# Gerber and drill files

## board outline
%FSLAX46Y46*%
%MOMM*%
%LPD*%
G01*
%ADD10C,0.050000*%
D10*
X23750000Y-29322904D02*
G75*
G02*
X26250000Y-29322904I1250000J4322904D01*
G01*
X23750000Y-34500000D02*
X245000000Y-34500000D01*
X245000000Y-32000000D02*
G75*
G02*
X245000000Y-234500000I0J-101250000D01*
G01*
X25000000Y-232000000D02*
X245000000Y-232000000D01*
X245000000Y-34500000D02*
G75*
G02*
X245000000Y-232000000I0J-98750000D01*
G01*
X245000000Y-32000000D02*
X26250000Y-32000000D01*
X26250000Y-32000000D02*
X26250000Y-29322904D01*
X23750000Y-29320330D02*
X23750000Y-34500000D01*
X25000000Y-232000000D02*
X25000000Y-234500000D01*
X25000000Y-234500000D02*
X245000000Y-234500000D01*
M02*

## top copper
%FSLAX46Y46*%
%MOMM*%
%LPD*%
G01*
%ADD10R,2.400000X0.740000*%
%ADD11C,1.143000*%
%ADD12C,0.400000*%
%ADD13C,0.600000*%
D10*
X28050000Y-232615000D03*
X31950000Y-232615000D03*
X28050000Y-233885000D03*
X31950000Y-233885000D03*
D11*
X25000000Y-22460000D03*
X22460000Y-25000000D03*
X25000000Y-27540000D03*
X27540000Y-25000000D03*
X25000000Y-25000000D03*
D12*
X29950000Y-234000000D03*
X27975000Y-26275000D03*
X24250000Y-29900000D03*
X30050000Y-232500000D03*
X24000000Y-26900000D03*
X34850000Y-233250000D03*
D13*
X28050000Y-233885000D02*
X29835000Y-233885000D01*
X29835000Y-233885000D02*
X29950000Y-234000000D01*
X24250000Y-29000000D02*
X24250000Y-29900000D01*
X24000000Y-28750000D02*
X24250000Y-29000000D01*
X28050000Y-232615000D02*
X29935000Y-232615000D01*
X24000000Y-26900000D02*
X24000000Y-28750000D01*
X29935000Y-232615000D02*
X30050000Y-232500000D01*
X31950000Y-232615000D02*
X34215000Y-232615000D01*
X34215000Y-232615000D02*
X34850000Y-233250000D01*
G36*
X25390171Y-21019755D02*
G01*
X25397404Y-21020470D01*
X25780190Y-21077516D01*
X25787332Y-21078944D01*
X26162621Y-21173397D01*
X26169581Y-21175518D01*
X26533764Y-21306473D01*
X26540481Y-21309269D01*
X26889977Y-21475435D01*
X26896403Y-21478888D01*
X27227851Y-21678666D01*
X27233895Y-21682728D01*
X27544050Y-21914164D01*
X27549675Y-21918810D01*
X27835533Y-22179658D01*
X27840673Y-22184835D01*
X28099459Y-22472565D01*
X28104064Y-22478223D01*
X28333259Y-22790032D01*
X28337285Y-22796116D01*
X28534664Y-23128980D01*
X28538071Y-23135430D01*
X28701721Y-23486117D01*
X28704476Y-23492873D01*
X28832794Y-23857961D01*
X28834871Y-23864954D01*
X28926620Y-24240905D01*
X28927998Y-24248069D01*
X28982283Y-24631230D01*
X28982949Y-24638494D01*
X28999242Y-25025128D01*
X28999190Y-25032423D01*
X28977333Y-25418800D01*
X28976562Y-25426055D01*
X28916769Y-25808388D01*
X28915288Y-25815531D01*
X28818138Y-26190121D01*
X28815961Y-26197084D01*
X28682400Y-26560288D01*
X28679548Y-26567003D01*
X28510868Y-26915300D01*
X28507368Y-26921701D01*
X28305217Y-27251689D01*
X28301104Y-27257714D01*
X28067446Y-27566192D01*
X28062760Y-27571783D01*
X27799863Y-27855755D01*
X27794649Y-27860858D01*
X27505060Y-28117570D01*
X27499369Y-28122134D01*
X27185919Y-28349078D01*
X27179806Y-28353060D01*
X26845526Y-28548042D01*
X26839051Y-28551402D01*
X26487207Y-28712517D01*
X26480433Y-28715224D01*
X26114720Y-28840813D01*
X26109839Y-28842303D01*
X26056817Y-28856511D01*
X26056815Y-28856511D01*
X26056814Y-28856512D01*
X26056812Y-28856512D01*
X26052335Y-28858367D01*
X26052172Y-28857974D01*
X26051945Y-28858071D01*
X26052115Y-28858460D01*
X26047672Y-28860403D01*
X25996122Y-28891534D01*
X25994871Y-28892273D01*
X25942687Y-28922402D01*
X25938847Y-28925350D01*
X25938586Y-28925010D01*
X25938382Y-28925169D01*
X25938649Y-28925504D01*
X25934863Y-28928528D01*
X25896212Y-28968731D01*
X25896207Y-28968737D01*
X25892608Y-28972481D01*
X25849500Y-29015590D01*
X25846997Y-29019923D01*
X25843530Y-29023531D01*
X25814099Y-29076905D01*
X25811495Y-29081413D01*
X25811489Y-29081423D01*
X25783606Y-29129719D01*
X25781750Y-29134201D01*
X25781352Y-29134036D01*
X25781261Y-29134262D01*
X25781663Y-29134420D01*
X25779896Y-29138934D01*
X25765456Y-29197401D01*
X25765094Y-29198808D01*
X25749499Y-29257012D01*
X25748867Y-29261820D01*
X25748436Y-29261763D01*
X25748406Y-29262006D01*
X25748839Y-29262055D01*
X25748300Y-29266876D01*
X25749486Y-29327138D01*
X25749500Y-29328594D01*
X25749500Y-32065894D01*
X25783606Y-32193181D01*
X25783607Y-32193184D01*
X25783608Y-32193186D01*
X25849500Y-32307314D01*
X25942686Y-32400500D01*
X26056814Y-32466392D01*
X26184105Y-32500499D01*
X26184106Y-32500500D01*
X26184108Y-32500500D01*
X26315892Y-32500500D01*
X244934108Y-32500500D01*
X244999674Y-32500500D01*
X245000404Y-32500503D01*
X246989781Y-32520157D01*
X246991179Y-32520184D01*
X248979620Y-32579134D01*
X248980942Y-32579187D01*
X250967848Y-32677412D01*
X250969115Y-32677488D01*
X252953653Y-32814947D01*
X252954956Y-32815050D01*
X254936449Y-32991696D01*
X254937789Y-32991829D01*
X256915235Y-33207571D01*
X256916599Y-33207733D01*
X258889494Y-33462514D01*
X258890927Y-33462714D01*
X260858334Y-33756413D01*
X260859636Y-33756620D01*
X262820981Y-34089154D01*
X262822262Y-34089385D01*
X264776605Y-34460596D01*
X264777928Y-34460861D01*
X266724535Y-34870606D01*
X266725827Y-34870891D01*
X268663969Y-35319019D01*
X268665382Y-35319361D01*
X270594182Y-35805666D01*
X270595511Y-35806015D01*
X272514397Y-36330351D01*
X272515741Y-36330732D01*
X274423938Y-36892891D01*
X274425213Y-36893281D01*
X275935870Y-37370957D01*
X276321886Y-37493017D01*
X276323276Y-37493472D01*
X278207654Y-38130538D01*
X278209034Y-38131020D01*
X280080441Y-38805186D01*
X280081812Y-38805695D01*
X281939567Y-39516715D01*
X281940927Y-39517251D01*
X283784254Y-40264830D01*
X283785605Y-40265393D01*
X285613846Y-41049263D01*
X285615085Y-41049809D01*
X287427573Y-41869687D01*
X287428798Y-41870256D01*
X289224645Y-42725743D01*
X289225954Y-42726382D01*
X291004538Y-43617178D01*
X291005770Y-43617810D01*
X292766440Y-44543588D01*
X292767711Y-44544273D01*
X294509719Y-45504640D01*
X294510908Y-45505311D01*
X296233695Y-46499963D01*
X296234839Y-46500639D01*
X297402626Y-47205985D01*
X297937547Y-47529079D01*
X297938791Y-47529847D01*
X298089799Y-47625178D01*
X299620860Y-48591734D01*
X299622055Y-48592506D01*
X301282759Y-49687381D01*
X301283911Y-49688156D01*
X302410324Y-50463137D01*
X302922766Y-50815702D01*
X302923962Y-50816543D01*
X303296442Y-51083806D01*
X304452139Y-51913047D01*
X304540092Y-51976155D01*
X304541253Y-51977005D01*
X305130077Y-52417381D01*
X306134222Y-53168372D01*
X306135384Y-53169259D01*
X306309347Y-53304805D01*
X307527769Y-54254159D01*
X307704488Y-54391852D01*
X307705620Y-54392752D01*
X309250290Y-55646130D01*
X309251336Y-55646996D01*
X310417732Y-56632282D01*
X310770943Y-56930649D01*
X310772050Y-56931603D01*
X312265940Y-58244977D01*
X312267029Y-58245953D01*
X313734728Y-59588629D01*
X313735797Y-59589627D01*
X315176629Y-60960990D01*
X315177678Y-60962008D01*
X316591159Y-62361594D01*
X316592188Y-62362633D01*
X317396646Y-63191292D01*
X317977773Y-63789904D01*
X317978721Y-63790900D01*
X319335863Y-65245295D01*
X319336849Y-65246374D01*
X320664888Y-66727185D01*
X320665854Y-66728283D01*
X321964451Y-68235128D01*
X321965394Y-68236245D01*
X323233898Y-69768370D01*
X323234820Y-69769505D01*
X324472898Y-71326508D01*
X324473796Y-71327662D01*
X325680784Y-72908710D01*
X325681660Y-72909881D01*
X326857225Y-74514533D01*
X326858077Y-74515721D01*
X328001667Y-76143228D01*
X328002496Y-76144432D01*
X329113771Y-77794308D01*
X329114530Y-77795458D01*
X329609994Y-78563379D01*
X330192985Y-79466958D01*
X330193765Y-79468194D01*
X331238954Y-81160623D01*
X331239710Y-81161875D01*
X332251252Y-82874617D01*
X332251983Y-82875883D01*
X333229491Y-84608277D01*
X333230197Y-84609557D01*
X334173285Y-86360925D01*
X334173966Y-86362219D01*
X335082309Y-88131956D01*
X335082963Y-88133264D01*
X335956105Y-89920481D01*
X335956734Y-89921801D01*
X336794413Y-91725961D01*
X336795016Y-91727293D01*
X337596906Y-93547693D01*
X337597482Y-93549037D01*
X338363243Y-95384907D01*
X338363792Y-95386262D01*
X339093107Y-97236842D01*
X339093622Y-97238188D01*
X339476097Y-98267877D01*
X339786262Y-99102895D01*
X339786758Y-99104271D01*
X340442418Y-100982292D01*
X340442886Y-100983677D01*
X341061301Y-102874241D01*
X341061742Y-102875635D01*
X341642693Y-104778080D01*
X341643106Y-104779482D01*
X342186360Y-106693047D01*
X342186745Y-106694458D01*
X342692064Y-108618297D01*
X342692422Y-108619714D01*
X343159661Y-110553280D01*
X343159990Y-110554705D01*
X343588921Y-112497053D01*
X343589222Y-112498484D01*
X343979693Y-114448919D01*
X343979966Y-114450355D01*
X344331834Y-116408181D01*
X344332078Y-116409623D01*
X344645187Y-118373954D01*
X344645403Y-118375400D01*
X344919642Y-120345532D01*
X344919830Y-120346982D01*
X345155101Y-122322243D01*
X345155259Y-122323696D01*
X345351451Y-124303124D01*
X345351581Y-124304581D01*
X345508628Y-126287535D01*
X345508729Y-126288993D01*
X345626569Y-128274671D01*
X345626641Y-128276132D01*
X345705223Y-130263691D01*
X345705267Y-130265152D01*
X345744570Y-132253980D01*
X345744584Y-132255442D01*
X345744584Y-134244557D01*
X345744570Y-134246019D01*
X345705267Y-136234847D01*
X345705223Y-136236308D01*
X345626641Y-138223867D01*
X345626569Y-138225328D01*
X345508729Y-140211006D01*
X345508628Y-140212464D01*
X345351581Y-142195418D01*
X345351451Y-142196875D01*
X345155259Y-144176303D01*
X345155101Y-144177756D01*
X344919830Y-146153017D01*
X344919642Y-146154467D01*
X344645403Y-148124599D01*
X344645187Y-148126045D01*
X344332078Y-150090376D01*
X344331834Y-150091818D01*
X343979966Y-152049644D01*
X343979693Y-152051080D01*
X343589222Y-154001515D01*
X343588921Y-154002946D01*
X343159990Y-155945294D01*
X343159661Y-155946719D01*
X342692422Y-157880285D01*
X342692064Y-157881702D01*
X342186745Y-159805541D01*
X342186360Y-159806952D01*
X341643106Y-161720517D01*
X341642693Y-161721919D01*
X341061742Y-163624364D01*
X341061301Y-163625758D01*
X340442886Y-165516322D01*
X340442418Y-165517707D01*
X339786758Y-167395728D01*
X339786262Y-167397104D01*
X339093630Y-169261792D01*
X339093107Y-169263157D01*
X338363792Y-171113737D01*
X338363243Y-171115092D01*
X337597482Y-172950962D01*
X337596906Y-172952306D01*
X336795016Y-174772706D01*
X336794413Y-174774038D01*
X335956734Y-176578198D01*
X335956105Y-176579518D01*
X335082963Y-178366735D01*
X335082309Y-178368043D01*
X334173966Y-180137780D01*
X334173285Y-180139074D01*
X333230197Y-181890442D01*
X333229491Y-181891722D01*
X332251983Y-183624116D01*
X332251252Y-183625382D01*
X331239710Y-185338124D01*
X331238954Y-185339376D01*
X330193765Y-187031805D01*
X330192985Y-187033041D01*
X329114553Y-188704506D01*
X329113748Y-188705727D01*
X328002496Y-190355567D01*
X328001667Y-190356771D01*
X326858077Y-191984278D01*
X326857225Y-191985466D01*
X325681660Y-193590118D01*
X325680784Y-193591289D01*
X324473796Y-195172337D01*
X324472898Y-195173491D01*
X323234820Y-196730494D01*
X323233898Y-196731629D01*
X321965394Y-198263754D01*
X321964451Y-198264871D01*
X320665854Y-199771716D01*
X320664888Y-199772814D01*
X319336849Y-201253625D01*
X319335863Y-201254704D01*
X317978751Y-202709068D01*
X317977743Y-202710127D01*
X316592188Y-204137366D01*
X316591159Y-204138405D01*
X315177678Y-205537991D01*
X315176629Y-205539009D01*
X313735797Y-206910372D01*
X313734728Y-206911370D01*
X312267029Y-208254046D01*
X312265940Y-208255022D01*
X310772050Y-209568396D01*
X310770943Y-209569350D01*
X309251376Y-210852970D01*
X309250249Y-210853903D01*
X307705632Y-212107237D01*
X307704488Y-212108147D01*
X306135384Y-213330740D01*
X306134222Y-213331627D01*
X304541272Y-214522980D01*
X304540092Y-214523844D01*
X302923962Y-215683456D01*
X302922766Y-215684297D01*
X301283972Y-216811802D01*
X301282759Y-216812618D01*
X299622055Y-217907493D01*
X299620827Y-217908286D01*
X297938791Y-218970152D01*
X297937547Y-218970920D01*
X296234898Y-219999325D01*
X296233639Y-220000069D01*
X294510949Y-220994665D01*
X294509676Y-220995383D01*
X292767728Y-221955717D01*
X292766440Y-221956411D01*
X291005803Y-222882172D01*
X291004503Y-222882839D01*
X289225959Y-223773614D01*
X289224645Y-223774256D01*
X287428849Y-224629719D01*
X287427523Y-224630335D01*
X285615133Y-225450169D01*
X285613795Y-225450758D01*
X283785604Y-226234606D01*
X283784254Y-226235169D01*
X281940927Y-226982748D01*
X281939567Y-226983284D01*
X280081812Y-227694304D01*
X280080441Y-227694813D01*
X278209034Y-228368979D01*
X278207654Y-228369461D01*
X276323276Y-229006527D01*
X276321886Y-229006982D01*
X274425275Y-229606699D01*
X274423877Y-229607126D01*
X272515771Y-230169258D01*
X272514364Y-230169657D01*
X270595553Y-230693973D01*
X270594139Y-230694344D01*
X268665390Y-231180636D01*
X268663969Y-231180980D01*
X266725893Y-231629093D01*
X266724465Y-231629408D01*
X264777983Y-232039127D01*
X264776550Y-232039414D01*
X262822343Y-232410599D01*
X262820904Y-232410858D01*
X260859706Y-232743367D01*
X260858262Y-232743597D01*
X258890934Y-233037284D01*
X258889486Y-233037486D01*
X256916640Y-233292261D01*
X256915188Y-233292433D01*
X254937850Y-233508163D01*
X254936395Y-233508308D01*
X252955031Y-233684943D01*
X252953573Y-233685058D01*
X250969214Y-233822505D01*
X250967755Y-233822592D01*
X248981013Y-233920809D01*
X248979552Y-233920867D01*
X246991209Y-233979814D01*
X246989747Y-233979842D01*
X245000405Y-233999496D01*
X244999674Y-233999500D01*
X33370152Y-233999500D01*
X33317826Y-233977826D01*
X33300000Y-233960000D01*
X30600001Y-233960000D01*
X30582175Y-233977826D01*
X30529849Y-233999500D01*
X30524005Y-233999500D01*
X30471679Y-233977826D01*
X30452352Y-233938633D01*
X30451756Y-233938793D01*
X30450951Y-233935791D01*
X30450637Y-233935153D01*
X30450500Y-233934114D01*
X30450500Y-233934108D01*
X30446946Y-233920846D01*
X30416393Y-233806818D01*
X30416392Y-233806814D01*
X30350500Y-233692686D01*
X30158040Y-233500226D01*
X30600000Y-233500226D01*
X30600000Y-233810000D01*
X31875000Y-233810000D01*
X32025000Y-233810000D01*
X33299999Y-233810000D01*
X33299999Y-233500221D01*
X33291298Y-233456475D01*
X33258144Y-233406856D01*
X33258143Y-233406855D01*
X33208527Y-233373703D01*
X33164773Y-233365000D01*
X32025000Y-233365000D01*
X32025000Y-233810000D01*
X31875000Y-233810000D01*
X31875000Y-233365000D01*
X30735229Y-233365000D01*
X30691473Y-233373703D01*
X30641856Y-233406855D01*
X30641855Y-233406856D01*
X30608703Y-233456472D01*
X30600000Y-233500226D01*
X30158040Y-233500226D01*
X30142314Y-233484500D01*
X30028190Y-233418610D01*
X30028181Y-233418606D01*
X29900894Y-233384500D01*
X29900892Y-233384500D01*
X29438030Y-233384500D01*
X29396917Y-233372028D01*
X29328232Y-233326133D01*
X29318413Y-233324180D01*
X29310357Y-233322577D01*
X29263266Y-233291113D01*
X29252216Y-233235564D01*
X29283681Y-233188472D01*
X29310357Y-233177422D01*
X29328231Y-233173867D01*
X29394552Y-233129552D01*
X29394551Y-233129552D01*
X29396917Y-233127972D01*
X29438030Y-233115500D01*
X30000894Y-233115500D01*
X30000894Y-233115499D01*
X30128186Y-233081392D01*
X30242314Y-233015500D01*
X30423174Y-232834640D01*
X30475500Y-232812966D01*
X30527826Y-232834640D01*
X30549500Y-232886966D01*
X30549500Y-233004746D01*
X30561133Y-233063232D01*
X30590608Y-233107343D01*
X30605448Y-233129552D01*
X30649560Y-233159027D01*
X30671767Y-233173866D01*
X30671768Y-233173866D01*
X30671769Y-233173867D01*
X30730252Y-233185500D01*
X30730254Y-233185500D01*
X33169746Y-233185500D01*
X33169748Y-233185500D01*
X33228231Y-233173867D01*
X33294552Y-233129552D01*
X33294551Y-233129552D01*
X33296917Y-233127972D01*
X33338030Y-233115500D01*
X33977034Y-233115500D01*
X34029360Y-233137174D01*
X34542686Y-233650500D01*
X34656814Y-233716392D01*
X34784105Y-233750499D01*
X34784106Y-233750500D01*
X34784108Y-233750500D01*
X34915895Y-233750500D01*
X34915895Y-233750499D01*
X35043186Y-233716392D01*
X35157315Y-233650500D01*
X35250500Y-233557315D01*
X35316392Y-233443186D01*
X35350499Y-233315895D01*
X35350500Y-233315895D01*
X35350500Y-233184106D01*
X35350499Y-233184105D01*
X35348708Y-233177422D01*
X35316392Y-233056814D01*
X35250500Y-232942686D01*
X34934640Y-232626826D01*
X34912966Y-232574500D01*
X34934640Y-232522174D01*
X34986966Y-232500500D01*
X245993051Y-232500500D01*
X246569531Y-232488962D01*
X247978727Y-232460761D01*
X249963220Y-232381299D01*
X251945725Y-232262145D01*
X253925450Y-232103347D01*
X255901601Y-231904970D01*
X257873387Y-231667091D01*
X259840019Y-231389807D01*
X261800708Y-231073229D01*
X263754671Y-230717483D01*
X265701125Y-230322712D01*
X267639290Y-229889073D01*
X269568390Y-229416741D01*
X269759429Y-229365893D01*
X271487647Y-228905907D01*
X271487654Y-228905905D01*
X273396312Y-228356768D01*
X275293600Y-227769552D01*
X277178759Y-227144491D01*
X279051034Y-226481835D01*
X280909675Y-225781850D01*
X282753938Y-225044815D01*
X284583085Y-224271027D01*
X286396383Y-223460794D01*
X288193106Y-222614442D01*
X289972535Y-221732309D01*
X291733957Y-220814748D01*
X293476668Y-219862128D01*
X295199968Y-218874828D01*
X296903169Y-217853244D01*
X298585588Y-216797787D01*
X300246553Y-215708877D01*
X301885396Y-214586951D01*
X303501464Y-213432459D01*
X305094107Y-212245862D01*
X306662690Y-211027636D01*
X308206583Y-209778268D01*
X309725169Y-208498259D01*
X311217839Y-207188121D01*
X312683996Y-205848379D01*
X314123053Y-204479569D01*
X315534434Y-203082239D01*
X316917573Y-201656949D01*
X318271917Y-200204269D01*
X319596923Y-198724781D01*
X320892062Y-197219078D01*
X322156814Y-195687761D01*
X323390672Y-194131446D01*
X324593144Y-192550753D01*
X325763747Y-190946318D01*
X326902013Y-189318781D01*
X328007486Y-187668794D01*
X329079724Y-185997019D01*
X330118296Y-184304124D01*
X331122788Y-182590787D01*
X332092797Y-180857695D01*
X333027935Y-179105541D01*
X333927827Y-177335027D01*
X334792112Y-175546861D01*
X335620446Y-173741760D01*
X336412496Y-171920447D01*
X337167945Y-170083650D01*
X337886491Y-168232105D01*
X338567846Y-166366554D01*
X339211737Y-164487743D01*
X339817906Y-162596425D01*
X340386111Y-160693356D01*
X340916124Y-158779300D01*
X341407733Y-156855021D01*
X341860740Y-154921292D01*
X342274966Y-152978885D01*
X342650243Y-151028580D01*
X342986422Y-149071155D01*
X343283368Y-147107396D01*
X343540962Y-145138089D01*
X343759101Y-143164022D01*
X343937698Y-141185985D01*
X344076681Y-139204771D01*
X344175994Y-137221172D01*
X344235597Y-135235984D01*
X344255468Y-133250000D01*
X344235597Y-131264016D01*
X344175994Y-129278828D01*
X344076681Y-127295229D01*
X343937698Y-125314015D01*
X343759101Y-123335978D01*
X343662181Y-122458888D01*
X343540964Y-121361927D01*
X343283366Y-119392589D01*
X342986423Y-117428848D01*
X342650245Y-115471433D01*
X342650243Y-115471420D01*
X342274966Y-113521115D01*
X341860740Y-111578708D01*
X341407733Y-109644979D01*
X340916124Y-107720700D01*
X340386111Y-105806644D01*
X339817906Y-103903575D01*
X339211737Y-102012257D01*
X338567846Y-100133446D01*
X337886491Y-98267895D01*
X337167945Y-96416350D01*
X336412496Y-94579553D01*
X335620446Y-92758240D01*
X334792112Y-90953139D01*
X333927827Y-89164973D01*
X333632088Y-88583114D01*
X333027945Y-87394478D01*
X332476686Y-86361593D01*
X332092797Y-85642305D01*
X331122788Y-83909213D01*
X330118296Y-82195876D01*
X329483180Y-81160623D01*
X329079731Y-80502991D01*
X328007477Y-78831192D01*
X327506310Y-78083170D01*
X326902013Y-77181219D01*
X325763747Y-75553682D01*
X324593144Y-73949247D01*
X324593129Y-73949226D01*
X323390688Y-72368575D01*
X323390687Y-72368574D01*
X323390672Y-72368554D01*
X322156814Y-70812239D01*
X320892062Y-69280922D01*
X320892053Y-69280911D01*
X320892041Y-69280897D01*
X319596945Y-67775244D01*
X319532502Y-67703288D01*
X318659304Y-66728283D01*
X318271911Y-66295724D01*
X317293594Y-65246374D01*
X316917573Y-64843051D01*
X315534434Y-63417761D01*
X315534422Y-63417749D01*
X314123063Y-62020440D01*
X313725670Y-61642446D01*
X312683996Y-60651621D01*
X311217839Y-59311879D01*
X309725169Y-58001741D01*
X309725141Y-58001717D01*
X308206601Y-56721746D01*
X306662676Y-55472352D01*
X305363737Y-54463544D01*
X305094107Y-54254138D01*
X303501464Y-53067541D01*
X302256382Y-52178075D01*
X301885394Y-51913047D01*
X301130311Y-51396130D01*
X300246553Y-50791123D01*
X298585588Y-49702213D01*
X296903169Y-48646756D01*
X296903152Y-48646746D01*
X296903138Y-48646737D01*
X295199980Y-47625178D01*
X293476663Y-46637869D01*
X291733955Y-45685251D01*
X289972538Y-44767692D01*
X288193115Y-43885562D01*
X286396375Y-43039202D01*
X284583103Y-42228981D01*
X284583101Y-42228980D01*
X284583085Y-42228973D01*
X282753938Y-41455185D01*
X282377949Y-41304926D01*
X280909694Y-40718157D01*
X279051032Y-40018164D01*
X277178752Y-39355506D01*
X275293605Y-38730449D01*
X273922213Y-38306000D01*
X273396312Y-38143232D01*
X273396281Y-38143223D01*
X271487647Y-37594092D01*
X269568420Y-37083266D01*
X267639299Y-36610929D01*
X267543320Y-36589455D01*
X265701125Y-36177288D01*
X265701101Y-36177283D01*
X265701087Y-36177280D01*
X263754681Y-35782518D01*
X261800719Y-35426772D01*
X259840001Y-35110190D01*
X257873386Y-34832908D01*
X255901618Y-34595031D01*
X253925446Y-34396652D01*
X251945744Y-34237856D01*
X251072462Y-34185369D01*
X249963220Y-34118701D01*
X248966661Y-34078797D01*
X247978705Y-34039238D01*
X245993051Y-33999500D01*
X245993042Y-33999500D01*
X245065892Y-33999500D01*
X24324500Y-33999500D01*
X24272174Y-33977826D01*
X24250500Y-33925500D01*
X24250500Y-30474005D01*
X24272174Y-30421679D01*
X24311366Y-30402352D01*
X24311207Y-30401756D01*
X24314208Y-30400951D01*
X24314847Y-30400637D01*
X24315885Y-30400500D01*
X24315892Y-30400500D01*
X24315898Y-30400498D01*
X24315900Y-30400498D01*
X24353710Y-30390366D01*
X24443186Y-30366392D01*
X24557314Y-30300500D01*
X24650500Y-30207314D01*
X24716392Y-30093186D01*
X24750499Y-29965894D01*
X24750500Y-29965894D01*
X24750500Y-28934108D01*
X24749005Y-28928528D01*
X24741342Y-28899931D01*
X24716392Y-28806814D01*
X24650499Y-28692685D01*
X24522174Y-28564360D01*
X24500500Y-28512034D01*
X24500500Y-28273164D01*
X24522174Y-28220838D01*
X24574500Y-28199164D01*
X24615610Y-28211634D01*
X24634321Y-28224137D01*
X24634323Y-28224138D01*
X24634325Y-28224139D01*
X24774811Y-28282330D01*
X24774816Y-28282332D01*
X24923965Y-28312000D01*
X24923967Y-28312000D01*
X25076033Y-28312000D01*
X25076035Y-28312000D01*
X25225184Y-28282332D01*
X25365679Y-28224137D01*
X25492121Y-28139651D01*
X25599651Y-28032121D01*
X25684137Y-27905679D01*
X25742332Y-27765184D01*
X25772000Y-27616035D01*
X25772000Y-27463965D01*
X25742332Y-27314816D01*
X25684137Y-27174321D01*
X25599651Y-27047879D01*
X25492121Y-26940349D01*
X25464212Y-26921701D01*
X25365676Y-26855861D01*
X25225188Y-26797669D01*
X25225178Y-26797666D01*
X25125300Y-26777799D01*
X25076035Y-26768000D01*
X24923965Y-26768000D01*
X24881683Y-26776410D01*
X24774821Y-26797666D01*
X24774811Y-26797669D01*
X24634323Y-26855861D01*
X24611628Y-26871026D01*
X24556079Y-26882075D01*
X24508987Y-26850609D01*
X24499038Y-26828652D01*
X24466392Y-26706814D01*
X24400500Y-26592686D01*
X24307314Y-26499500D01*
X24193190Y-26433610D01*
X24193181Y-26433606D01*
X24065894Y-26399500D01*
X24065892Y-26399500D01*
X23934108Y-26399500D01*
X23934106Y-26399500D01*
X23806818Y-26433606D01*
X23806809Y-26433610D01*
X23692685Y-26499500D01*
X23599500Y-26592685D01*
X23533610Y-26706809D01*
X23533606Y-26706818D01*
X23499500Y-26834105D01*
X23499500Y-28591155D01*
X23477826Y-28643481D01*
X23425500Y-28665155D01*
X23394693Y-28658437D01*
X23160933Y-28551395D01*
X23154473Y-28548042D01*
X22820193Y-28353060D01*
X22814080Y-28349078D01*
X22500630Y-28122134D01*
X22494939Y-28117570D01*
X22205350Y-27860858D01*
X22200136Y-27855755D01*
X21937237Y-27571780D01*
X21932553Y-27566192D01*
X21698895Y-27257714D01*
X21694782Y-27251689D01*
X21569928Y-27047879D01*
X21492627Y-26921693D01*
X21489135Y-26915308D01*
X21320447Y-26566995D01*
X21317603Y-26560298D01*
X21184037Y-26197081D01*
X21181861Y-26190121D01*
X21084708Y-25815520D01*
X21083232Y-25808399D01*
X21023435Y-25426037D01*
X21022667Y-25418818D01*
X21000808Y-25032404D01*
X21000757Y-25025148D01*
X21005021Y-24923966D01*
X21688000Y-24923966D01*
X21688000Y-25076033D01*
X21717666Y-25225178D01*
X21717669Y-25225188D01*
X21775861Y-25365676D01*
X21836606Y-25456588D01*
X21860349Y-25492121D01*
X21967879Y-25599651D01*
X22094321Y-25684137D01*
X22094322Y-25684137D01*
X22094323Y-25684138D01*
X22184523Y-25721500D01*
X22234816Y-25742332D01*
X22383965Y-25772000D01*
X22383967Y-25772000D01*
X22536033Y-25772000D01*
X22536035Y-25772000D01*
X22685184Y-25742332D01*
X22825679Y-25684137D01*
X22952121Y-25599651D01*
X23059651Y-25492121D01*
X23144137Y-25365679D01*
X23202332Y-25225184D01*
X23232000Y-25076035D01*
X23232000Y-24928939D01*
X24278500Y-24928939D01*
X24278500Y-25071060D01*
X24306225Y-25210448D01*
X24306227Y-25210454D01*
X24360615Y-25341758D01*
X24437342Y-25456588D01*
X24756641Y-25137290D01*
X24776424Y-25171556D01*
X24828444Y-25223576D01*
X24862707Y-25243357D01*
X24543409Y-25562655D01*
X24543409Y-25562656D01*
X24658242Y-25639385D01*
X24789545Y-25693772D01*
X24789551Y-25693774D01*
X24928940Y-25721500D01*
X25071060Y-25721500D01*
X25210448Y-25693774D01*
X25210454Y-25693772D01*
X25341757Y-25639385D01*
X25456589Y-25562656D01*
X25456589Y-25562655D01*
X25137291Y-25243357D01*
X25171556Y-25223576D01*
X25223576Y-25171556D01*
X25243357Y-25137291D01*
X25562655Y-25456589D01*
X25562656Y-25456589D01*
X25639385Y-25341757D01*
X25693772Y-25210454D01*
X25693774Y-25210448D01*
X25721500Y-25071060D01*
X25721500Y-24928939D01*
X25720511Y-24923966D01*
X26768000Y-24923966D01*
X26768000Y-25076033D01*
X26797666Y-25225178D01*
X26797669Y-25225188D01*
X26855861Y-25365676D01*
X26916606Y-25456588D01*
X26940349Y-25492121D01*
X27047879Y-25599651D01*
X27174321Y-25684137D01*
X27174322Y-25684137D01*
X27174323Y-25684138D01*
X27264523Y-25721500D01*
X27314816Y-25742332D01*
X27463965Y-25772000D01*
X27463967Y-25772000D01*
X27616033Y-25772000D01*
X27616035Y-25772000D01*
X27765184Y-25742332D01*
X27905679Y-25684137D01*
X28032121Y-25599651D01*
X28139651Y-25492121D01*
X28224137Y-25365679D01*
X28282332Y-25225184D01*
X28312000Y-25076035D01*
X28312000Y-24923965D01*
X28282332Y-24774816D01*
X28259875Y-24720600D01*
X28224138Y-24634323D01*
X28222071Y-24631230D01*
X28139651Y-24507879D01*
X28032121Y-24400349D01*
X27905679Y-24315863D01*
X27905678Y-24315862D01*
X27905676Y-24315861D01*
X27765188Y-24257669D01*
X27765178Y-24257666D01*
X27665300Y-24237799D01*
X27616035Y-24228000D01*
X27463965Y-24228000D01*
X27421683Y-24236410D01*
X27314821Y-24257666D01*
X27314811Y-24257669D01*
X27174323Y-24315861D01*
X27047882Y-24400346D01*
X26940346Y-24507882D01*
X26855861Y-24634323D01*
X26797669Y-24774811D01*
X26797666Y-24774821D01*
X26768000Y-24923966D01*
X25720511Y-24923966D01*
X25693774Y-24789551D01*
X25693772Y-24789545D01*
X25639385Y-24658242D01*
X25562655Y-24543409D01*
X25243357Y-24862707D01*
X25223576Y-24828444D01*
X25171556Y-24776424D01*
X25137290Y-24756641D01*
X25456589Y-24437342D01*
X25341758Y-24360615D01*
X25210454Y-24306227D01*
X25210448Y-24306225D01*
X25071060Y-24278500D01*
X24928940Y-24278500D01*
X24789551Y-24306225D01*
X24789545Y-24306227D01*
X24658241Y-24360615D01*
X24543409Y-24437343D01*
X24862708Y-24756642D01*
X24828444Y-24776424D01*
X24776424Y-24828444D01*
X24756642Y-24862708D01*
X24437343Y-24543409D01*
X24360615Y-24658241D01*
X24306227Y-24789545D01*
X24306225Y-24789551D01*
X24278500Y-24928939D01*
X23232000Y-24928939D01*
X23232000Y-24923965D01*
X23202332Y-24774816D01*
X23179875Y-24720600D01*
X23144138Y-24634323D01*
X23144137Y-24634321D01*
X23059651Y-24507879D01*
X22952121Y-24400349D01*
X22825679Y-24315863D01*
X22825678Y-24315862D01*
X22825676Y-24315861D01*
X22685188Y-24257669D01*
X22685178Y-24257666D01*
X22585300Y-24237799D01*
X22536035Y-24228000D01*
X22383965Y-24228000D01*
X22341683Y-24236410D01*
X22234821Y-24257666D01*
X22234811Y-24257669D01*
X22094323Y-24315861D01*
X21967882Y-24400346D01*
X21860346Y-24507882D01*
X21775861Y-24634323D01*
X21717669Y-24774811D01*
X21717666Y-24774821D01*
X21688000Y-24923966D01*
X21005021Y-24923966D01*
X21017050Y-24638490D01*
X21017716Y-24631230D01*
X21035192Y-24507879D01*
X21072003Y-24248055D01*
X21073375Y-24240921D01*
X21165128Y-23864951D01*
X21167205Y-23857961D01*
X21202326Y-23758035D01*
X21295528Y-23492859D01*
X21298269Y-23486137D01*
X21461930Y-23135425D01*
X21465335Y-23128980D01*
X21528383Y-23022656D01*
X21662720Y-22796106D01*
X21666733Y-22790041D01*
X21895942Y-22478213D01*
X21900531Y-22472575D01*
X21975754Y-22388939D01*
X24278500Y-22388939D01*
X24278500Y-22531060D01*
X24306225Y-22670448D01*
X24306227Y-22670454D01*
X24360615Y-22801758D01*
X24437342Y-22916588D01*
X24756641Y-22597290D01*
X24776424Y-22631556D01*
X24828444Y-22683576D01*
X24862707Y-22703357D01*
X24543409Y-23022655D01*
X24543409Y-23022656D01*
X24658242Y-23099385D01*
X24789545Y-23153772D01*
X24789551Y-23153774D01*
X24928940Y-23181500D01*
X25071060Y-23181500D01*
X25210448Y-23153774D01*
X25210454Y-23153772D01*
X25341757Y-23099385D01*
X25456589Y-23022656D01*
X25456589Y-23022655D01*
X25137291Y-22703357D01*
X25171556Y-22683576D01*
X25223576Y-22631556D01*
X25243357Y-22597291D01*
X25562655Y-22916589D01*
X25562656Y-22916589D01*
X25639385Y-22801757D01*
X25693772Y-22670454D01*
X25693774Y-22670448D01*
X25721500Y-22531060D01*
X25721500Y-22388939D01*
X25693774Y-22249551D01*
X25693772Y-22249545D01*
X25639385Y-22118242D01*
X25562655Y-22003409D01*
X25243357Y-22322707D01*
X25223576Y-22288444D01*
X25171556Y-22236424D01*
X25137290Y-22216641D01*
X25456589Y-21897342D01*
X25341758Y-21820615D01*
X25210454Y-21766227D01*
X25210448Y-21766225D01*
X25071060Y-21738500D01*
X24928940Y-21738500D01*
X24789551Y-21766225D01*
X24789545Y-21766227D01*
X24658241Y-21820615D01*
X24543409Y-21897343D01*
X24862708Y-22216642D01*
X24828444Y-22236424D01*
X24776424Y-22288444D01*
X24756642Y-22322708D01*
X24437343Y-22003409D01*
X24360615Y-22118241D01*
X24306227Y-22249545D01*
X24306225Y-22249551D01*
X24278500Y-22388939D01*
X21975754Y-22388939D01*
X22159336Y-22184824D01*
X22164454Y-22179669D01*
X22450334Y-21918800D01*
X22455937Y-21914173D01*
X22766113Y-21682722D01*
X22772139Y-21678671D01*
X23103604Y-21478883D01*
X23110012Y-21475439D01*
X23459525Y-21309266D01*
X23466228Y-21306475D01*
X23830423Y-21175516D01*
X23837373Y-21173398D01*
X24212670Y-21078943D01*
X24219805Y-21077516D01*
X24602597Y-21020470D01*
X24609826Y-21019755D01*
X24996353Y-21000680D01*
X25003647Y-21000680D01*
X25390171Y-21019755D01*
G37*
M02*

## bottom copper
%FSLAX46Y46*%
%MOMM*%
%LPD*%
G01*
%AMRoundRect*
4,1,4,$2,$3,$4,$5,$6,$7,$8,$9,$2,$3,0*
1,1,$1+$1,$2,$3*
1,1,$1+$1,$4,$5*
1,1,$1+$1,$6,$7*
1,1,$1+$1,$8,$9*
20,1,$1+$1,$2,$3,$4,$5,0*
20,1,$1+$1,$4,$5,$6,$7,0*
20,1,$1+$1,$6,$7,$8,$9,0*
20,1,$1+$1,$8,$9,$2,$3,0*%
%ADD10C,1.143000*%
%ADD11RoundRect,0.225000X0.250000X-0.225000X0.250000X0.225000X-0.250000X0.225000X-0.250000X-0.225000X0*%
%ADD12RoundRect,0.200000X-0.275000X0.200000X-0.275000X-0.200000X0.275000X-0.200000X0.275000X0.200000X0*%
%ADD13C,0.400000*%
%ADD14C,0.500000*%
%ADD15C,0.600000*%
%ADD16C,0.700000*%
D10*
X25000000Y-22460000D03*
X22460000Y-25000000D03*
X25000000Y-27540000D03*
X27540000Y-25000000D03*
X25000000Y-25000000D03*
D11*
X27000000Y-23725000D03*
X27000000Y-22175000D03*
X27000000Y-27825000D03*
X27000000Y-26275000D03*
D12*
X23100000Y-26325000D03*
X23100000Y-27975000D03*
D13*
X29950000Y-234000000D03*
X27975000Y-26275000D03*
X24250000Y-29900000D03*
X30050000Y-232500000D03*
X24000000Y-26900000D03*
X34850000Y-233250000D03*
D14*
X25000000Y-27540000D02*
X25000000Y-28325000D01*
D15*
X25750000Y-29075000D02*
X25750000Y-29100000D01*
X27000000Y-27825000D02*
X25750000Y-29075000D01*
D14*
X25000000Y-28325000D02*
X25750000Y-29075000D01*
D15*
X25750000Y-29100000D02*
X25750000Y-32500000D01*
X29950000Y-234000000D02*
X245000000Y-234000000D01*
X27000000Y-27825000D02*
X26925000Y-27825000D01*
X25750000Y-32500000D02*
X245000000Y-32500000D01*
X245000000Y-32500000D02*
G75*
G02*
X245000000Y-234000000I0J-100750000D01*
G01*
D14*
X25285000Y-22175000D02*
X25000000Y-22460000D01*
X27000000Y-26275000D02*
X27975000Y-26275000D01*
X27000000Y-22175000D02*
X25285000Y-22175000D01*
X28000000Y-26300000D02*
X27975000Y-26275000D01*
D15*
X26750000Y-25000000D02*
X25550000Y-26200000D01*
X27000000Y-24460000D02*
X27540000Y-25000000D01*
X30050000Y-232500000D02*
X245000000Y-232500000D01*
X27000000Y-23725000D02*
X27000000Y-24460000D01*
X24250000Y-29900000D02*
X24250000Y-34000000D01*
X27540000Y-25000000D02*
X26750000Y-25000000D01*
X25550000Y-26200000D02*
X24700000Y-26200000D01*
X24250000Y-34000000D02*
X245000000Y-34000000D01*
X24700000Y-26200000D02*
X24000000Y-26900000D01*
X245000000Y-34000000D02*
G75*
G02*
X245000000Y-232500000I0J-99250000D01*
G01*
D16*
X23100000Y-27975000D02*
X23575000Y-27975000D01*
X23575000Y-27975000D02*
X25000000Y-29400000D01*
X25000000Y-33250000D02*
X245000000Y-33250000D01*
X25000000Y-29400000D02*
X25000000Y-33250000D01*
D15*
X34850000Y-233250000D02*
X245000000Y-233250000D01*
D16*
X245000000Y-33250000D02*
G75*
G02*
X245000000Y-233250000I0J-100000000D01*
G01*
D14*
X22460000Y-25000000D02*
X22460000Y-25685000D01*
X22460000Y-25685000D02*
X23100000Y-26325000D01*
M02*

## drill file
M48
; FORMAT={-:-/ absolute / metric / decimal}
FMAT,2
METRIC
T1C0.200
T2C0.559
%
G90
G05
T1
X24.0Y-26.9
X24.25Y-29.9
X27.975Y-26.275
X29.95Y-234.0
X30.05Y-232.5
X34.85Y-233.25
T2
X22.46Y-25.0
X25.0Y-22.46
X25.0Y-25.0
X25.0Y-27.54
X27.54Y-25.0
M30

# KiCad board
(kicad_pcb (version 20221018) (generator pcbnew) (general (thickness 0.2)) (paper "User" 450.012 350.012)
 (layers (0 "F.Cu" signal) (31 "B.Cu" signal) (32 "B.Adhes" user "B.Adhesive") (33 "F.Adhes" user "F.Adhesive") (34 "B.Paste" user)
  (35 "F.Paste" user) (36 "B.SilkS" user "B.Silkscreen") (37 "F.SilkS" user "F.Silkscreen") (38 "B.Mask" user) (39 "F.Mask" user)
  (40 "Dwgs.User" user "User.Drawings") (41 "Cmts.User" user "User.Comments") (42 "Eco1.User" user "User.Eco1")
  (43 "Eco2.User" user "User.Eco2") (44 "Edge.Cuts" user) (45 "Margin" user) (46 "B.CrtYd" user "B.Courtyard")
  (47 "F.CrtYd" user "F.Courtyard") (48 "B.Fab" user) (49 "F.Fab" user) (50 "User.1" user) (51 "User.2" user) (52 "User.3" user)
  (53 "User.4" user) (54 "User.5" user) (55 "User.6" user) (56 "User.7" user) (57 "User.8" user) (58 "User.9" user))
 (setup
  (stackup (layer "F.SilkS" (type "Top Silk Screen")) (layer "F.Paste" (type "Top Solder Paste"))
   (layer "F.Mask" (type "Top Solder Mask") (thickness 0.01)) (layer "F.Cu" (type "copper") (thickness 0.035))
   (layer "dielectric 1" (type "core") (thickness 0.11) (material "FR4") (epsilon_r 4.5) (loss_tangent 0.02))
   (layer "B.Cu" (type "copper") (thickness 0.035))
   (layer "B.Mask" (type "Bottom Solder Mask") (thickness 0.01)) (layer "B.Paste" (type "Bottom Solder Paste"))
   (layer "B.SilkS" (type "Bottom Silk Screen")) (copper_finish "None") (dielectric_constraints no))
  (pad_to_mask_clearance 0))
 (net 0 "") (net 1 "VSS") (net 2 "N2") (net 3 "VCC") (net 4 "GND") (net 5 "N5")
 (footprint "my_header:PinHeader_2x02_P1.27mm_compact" (layer "F.Cu") (at 30 233.25)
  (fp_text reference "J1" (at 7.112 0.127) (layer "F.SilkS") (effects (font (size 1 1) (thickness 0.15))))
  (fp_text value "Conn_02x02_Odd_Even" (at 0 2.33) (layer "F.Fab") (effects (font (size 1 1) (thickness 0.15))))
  (pad "1" smd rect (at -1.95 -0.635) (size 2.4 0.74) (layers "F.Cu" "F.Paste" "F.Mask") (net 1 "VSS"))
  (pad "2" smd rect (at 1.95 -0.635) (size 2.4 0.74) (layers "F.Cu" "F.Paste" "F.Mask") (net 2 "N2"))
  (pad "3" smd rect (at -1.95 0.635) (size 2.4 0.74) (layers "F.Cu" "F.Paste" "F.Mask") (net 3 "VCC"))
  (pad "4" smd rect (at 1.95 0.635) (size 2.4 0.74) (layers "F.Cu" "F.Paste" "F.Mask") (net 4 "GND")))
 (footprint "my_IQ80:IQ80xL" (layer "F.Cu") (at 25 25 90)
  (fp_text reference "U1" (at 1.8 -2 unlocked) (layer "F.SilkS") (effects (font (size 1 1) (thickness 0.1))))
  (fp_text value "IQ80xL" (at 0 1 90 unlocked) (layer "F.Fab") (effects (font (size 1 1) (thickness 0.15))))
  (pad "1" thru_hole circle (at 2.54 0 90) (size 1.143 1.143) (drill 0.5588) (layers "*.Cu" "*.Mask") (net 4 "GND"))
  (pad "2" thru_hole circle (at 0 -2.54 90) (size 1.143 1.143) (drill 0.5588) (layers "*.Cu" "*.Mask") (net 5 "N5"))
  (pad "3" thru_hole circle (at -2.54 0 90) (size 1.143 1.143) (drill 0.5588) (layers "*.Cu" "*.Mask") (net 3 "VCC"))
  (pad "4" thru_hole circle (at 0 2.54 90) (size 1.143 1.143) (drill 0.5588) (layers "*.Cu" "*.Mask") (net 1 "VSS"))
  (pad "5" thru_hole circle (at 0 0 90) (size 1.143 1.143) (drill 0.5588) (layers "*.Cu" "*.Mask") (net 4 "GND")))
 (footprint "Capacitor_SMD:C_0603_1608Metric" (layer "B.Cu") (at 27 22.95 90)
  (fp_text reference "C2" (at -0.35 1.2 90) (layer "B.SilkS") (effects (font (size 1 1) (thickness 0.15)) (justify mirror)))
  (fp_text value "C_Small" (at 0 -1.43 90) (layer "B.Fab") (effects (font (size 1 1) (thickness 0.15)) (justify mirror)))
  (pad "1" smd roundrect (at -0.775 0 90) (size 0.9 0.95) (layers "B.Cu" "B.Paste" "B.Mask") (roundrect_rratio 0.25) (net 1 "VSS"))
  (pad "2" smd roundrect (at 0.775 0 90) (size 0.9 0.95) (layers "B.Cu" "B.Paste" "B.Mask") (roundrect_rratio 0.25) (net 4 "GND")))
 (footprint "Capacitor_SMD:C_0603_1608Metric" (layer "B.Cu") (at 27 27.05 90)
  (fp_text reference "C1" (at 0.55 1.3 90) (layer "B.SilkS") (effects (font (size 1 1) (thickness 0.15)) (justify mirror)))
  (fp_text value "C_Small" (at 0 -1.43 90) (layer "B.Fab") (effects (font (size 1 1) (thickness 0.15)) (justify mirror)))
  (pad "1" smd roundrect (at -0.775 0 90) (size 0.9 0.95) (layers "B.Cu" "B.Paste" "B.Mask") (roundrect_rratio 0.25) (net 3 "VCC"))
  (pad "2" smd roundrect (at 0.775 0 90) (size 0.9 0.95) (layers "B.Cu" "B.Paste" "B.Mask") (roundrect_rratio 0.25) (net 4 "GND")))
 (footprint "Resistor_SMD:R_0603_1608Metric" (layer "B.Cu") (at 23.1 27.15 -90)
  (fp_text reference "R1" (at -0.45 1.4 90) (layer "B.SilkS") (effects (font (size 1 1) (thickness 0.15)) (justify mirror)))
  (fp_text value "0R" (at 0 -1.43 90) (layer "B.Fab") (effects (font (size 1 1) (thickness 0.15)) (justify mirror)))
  (pad "1" smd roundrect (at -0.825 0 270) (size 0.8 0.95) (layers "B.Cu" "B.Paste" "B.Mask") (roundrect_rratio 0.25) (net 5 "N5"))
  (pad "2" smd roundrect (at 0.825 0 270) (size 0.8 0.95) (layers "B.Cu" "B.Paste" "B.Mask") (roundrect_rratio 0.25) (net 2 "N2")))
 (gr_arc (start 23.75 29.322904) (mid 25 20.5) (end 26.25 29.322904) (stroke (width 0.05) (type solid)) (layer "Edge.Cuts"))
 (gr_line (start 23.75 34.5) (end 245 34.5) (stroke (width 0.05) (type solid)) (layer "Edge.Cuts"))
 (gr_arc (start 245 32) (mid 346.25 133.25) (end 245 234.5) (stroke (width 0.05) (type solid)) (layer "Edge.Cuts"))
 (gr_line (start 25 232) (end 245 232) (stroke (width 0.05) (type solid)) (layer "Edge.Cuts"))
 (gr_arc (start 245 34.5) (mid 343.75 133.25) (end 245 232) (stroke (width 0.05) (type solid)) (layer "Edge.Cuts"))
 (gr_line (start 245 32) (end 26.25 32) (stroke (width 0.05) (type solid)) (layer "Edge.Cuts"))
 (gr_line (start 26.25 32) (end 26.25 29.322904) (stroke (width 0.05) (type solid)) (layer "Edge.Cuts"))
 (gr_line (start 23.75 29.32033) (end 23.75 34.5) (stroke (width 0.05) (type solid)) (layer "Edge.Cuts"))
 (gr_line (start 25 232) (end 25 234.5) (stroke (width 0.05) (type solid)) (layer "Edge.Cuts"))
 (gr_line (start 25 234.5) (end 245 234.5) (stroke (width 0.05) (type solid)) (layer "Edge.Cuts"))
 (segment (start 28.05 233.885) (end 29.835 233.885) (width 0.6) (layer "F.Cu") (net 3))
 (segment (start 29.835 233.885) (end 29.95 234) (width 0.6) (layer "F.Cu") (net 3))
 (via (at 29.95 234) (size 0.4) (drill 0.2) (layers "F.Cu" "B.Cu") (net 3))
 (segment (start 25 27.54) (end 25 28.325) (width 0.5) (layer "B.Cu") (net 3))
 (segment (start 25.75 29.075) (end 25.75 29.1) (width 0.6) (layer "B.Cu") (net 3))
 (segment (start 27 27.825) (end 25.75 29.075) (width 0.6) (layer "B.Cu") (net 3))
 (segment (start 25 28.325) (end 25.75 29.075) (width 0.5) (layer "B.Cu") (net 3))
 (segment (start 25.75 29.1) (end 25.75 32.5) (width 0.6) (layer "B.Cu") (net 3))
 (segment (start 29.95 234) (end 245 234) (width 0.6) (layer "B.Cu") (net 3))
 (segment (start 27 27.825) (end 26.925 27.825) (width 0.6) (layer "B.Cu") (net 3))
 (segment (start 25.75 32.5) (end 245 32.5) (width 0.6) (layer "B.Cu") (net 3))
 (arc (start 245 32.5) (mid 345.75 133.25) (end 245 234) (width 0.6) (layer "B.Cu") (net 3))
 (via (at 27.975 26.275) (size 0.4) (drill 0.2) (layers "F.Cu" "B.Cu") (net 4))
 (segment (start 25.285 22.175) (end 25 22.46) (width 0.5) (layer "B.Cu") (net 4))
 (segment (start 27 26.275) (end 27.975 26.275) (width 0.5) (layer "B.Cu") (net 4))
 (segment (start 27 22.175) (end 25.285 22.175) (width 0.5) (layer "B.Cu") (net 4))
 (segment (start 28 26.3) (end 27.975 26.275) (width 0.5) (layer "B.Cu") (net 4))
 (segment (start 24.25 29) (end 24.25 29.9) (width 0.6) (layer "F.Cu") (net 1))
 (segment (start 24 28.75) (end 24.25 29) (width 0.6) (layer "F.Cu") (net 1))
 (segment (start 28.05 232.615) (end 29.935 232.615) (width 0.6) (layer "F.Cu") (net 1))
 (segment (start 24 26.9) (end 24 28.75) (width 0.6) (layer "F.Cu") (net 1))
 (segment (start 29.935 232.615) (end 30.05 232.5) (width 0.6) (layer "F.Cu") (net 1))
 (via (at 24.25 29.9) (size 0.4) (drill 0.2) (layers "F.Cu" "B.Cu") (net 1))
 (via (at 30.05 232.5) (size 0.4) (drill 0.2) (layers "F.Cu" "B.Cu") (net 1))
 (via (at 24 26.9) (size 0.4) (drill 0.2) (layers "F.Cu" "B.Cu") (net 1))
 (segment (start 26.75 25) (end 25.55 26.2) (width 0.6) (layer "B.Cu") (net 1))
 (segment (start 27 24.46) (end 27.54 25) (width 0.6) (layer "B.Cu") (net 1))
 (segment (start 30.05 232.5) (end 245 232.5) (width 0.6) (layer "B.Cu") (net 1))
 (segment (start 27 23.725) (end 27 24.46) (width 0.6) (layer "B.Cu") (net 1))
 (segment (start 24.25 29.9) (end 24.25 34) (width 0.6) (layer "B.Cu") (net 1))
 (segment (start 27.54 25) (end 26.75 25) (width 0.6) (layer "B.Cu") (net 1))
 (segment (start 25.55 26.2) (end 24.7 26.2) (width 0.6) (layer "B.Cu") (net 1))
 (segment (start 24.25 34) (end 245 34) (width 0.6) (layer "B.Cu") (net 1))
 (segment (start 24.7 26.2) (end 24 26.9) (width 0.6) (layer "B.Cu") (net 1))
 (arc (start 245 34) (mid 344.25 133.25) (end 245 232.5) (width 0.6) (layer "B.Cu") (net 1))
 (segment (start 31.95 232.615) (end 34.215 232.615) (width 0.6) (layer "F.Cu") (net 2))
 (segment (start 34.215 232.615) (end 34.85 233.25) (width 0.6) (layer "F.Cu") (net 2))
 (via (at 34.85 233.25) (size 0.4) (drill 0.2) (layers "F.Cu" "B.Cu") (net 2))
 (segment (start 23.1 27.975) (end 23.575 27.975) (width 0.7) (layer "B.Cu") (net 2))
 (segment (start 23.575 27.975) (end 25 29.4) (width 0.7) (layer "B.Cu") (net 2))
 (segment (start 25 33.25) (end 245 33.25) (width 0.7) (layer "B.Cu") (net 2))
 (segment (start 25 29.4) (end 25 33.25) (width 0.7) (layer "B.Cu") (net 2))
 (segment (start 34.85 233.25) (end 245 233.25) (width 0.6) (layer "B.Cu") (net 2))
 (arc (start 245 33.25) (mid 345 133.25) (end 245 233.25) (width 0.7) (layer "B.Cu") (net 2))
 (segment (start 22.46 25) (end 22.46 25.685) (width 0.5) (layer "B.Cu") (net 5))
 (segment (start 22.46 25.685) (end 23.1 26.325) (width 0.5) (layer "B.Cu") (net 5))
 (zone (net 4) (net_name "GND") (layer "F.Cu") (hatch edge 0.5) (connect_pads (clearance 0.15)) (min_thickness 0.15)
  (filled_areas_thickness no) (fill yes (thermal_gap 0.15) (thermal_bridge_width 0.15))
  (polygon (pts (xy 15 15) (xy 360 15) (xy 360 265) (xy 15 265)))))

